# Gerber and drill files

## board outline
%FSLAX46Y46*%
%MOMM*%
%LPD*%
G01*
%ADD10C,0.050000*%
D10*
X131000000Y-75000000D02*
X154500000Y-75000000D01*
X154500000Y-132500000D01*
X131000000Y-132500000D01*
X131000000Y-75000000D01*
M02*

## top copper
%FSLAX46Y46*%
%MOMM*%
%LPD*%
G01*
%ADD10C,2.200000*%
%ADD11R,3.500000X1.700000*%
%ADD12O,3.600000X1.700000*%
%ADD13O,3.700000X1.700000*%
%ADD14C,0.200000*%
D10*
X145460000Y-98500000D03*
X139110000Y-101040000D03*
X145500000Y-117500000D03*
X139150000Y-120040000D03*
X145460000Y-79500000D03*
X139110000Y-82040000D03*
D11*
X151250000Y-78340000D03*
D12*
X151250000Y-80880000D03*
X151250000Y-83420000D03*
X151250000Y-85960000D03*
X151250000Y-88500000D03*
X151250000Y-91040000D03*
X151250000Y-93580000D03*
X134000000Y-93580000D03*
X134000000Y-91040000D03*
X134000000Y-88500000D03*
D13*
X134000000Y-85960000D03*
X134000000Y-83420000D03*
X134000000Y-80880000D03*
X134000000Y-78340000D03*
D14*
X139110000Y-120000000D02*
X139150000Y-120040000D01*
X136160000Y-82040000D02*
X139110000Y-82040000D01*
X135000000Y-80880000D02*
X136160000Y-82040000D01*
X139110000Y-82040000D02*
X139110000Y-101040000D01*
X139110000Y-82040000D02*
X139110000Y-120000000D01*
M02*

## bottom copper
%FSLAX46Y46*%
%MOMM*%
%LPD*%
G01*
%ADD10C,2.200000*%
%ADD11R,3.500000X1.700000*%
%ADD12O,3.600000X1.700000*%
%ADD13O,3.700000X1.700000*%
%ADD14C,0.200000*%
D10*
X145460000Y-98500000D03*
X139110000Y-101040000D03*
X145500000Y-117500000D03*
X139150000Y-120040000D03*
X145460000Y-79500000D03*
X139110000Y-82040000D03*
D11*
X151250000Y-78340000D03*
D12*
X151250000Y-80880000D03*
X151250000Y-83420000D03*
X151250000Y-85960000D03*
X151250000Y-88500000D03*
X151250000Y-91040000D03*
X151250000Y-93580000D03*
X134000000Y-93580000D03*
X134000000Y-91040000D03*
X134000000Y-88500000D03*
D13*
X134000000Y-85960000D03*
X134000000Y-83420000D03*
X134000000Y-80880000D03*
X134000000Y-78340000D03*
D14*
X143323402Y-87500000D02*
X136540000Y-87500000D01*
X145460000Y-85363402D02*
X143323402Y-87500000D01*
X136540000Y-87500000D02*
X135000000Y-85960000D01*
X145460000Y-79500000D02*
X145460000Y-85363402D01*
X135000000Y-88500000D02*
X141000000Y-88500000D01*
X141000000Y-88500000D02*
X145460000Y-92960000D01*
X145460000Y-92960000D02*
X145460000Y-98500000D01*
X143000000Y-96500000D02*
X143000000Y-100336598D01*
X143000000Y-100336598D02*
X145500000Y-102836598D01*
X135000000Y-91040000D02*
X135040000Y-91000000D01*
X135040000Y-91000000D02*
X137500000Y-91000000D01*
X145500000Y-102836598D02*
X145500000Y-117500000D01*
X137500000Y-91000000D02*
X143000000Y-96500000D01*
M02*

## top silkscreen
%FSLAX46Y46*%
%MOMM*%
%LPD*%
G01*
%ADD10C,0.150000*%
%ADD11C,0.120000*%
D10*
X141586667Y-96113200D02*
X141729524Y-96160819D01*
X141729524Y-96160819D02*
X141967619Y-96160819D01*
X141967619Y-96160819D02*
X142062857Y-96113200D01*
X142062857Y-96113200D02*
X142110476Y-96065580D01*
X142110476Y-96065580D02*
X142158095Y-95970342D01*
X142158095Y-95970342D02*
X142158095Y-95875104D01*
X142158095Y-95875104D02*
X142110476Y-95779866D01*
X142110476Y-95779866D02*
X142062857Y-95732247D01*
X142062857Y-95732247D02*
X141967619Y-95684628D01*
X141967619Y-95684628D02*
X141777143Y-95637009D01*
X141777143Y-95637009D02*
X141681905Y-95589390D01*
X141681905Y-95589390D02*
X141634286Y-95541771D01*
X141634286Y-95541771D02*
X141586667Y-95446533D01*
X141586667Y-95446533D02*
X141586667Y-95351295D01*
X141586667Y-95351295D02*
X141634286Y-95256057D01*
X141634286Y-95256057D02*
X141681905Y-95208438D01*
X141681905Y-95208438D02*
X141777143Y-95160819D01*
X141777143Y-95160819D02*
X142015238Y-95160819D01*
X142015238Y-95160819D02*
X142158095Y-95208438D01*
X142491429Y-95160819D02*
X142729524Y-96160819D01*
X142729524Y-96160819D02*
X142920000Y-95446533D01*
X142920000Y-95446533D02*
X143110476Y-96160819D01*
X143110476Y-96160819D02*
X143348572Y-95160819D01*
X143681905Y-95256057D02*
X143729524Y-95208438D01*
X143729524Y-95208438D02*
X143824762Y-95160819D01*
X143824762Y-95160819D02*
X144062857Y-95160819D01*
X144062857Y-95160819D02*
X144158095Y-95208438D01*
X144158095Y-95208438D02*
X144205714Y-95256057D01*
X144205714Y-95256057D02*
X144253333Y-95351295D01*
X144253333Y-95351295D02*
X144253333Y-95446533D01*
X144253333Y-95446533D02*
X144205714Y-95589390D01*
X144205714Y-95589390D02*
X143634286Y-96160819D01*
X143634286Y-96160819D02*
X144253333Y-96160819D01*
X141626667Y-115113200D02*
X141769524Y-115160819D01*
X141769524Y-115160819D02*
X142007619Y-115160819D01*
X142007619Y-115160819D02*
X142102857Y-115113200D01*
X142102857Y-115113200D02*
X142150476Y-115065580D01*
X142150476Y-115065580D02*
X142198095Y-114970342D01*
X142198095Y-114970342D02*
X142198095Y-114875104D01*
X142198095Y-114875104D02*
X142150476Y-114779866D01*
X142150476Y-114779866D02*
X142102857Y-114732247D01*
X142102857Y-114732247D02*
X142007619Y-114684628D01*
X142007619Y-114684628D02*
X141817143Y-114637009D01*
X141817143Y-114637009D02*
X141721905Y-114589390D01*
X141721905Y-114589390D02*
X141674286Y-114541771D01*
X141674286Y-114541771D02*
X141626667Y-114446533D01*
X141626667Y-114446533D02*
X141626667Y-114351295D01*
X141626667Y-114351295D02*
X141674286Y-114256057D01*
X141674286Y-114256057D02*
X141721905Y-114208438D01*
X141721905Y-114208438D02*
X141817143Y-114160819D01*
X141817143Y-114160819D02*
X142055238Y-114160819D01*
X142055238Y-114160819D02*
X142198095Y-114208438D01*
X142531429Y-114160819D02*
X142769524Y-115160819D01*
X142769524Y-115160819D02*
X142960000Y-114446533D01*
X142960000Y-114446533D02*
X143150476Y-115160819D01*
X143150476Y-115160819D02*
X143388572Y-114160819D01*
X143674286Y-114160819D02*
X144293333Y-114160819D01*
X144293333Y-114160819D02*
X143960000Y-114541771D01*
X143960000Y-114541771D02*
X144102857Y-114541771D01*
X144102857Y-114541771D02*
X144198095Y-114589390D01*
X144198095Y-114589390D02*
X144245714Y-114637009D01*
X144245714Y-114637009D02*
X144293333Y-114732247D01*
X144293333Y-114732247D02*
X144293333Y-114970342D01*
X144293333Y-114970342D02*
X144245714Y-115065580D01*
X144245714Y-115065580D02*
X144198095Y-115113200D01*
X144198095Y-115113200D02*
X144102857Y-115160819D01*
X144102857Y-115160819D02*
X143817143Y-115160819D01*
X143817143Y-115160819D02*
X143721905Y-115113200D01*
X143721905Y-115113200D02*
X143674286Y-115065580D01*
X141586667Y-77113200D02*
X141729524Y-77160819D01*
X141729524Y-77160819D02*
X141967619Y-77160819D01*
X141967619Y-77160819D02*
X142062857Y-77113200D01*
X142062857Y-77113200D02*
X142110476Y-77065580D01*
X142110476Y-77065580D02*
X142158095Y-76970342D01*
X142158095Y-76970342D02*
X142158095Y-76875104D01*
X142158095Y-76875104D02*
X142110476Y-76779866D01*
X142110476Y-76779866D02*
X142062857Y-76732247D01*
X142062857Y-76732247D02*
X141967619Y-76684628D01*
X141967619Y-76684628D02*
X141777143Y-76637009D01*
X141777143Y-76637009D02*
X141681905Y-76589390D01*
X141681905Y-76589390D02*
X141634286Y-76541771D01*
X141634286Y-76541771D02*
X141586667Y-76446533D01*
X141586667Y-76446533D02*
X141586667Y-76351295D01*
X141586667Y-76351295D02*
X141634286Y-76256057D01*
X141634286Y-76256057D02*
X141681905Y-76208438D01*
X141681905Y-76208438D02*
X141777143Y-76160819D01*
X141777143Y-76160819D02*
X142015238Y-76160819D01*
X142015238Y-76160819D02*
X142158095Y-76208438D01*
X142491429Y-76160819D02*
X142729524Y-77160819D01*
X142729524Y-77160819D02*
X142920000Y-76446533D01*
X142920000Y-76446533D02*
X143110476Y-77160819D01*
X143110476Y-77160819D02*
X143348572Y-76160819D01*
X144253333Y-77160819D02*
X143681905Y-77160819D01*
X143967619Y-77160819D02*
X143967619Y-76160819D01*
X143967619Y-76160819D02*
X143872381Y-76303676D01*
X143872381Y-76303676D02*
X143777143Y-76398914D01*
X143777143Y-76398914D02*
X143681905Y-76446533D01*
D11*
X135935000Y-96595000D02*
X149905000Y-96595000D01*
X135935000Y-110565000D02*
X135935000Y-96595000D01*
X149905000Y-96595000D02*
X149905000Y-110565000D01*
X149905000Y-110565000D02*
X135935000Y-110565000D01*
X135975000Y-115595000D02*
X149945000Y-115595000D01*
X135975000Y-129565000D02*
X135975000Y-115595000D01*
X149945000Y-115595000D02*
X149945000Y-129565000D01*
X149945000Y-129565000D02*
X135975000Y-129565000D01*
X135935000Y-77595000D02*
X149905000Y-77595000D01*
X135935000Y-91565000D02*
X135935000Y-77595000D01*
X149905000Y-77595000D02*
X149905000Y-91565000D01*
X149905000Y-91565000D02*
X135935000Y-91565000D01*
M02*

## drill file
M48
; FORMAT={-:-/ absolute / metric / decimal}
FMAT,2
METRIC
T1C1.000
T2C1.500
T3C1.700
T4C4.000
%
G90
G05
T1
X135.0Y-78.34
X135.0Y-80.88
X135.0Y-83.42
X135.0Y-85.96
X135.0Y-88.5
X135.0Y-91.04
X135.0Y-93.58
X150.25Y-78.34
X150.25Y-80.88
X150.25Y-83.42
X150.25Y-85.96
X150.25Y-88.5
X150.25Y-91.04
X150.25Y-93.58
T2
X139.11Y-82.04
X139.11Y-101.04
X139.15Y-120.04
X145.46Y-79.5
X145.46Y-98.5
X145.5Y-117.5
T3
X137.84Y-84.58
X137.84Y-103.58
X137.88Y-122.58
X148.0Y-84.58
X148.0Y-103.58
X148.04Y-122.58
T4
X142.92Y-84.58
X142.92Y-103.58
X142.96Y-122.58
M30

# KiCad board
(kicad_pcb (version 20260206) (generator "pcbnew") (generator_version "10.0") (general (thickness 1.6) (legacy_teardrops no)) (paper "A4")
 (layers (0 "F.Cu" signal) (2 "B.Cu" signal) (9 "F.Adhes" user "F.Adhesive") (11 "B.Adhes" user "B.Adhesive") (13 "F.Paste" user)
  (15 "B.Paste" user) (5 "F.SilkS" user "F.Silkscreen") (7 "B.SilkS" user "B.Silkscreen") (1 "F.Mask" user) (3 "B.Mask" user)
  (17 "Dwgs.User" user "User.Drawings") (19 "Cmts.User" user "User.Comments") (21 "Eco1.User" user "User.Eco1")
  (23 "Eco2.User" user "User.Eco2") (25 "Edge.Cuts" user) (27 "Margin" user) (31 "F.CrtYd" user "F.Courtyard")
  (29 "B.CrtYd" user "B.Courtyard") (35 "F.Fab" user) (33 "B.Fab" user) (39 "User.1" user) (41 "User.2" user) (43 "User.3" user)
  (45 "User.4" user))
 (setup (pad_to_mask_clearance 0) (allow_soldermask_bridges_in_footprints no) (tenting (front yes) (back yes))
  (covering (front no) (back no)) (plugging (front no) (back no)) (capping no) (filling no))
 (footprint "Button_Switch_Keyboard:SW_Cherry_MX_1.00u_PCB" (layer "F.Cu") (at 145.46 98.5)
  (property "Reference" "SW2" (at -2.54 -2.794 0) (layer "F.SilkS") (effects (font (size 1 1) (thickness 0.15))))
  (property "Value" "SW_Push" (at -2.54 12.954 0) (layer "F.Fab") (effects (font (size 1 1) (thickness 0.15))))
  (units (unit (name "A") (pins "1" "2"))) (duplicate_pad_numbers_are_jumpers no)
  (fp_line (start -9.525 -1.905) (end 4.445 -1.905) (stroke (width 0.12) (type solid)) (layer "F.SilkS"))
  (fp_line (start -9.525 12.065) (end -9.525 -1.905) (stroke (width 0.12) (type solid)) (layer "F.SilkS"))
  (fp_line (start 4.445 -1.905) (end 4.445 12.065) (stroke (width 0.12) (type solid)) (layer "F.SilkS"))
  (fp_line (start 4.445 12.065) (end -9.525 12.065) (stroke (width 0.12) (type solid)) (layer "F.SilkS"))
  (pad "" np_thru_hole circle (at -7.62 5.08) (size 1.7 1.7) (drill 1.7) (layers "*.Cu" "*.Mask"))
  (pad "" np_thru_hole circle (at -2.54 5.08) (size 4 4) (drill 4) (layers "*.Cu" "*.Mask"))
  (pad "" np_thru_hole circle (at 2.54 5.08) (size 1.7 1.7) (drill 1.7) (layers "*.Cu" "*.Mask"))
  (pad "1" thru_hole circle (at 0 0) (size 2.2 2.2) (drill 1.5) (layers "*.Cu" "*.Mask") (remove_unused_layers no)
   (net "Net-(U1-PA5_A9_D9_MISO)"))
  (pad "2" thru_hole circle (at -6.35 2.54) (size 2.2 2.2) (drill 1.5) (layers "*.Cu" "*.Mask") (remove_unused_layers no) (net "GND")))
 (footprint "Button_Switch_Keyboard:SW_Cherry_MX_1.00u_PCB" (layer "F.Cu") (at 145.5 117.5)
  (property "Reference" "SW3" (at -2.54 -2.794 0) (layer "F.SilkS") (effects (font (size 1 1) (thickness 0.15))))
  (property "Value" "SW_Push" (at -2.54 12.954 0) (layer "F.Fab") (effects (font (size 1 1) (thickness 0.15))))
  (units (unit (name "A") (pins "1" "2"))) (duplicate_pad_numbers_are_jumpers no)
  (fp_line (start -9.525 -1.905) (end 4.445 -1.905) (stroke (width 0.12) (type solid)) (layer "F.SilkS"))
  (fp_line (start -9.525 12.065) (end -9.525 -1.905) (stroke (width 0.12) (type solid)) (layer "F.SilkS"))
  (fp_line (start 4.445 -1.905) (end 4.445 12.065) (stroke (width 0.12) (type solid)) (layer "F.SilkS"))
  (fp_line (start 4.445 12.065) (end -9.525 12.065) (stroke (width 0.12) (type solid)) (layer "F.SilkS"))
  (pad "" np_thru_hole circle (at -7.62 5.08) (size 1.7 1.7) (drill 1.7) (layers "*.Cu" "*.Mask"))
  (pad "" np_thru_hole circle (at -2.54 5.08) (size 4 4) (drill 4) (layers "*.Cu" "*.Mask"))
  (pad "" np_thru_hole circle (at 2.54 5.08) (size 1.7 1.7) (drill 1.7) (layers "*.Cu" "*.Mask"))
  (pad "1" thru_hole circle (at 0 0) (size 2.2 2.2) (drill 1.5) (layers "*.Cu" "*.Mask") (remove_unused_layers no)
   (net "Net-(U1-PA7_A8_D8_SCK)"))
  (pad "2" thru_hole circle (at -6.35 2.54) (size 2.2 2.2) (drill 1.5) (layers "*.Cu" "*.Mask") (remove_unused_layers no) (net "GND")))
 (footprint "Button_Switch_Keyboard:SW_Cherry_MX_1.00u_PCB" (layer "F.Cu") (at 145.46 79.5)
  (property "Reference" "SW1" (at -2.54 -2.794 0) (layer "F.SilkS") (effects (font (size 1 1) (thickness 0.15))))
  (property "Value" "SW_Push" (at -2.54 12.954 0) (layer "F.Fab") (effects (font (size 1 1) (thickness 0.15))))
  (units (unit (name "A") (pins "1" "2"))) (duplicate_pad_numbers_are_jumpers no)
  (fp_line (start -9.525 -1.905) (end 4.445 -1.905) (stroke (width 0.12) (type solid)) (layer "F.SilkS"))
  (fp_line (start -9.525 12.065) (end -9.525 -1.905) (stroke (width 0.12) (type solid)) (layer "F.SilkS"))
  (fp_line (start 4.445 -1.905) (end 4.445 12.065) (stroke (width 0.12) (type solid)) (layer "F.SilkS"))
  (fp_line (start 4.445 12.065) (end -9.525 12.065) (stroke (width 0.12) (type solid)) (layer "F.SilkS"))
  (pad "" np_thru_hole circle (at -7.62 5.08) (size 1.7 1.7) (drill 1.7) (layers "*.Cu" "*.Mask"))
  (pad "" np_thru_hole circle (at -2.54 5.08) (size 4 4) (drill 4) (layers "*.Cu" "*.Mask"))
  (pad "" np_thru_hole circle (at 2.54 5.08) (size 1.7 1.7) (drill 1.7) (layers "*.Cu" "*.Mask"))
  (pad "1" thru_hole circle (at 0 0) (size 2.2 2.2) (drill 1.5) (layers "*.Cu" "*.Mask") (remove_unused_layers no)
   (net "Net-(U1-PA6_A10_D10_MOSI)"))
  (pad "2" thru_hole circle (at -6.35 2.54) (size 2.2 2.2) (drill 1.5) (layers "*.Cu" "*.Mask") (remove_unused_layers no) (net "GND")))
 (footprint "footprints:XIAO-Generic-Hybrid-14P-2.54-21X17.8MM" (layer "B.Cu") (at 142.625 85.96 180)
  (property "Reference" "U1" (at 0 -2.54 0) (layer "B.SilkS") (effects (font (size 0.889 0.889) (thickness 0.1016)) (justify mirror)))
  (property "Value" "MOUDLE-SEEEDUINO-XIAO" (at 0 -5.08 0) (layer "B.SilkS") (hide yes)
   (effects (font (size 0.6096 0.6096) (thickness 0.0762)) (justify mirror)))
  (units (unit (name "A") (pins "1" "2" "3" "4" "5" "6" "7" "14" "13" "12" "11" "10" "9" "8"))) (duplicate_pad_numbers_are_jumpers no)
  (pad "1" thru_hole rect (at -7.625 7.62 180) (size 3.5 1.7) (drill 1 (offset -1 0)) (layers "*.Cu" "*.Mask") (remove_unused_layers no)
   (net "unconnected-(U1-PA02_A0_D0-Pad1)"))
  (pad "2" thru_hole oval (at -7.625 5.08 180) (size 3.6 1.7) (drill 1 (offset -1 0)) (layers "*.Cu" "*.Mask") (remove_unused_layers no)
   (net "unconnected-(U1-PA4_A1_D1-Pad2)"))
  (pad "3" thru_hole oval (at -7.625 2.54 180) (size 3.6 1.7) (drill 1 (offset -1 0)) (layers "*.Cu" "*.Mask") (remove_unused_layers no)
   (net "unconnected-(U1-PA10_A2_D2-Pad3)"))
  (pad "4" thru_hole oval (at -7.625 0 180) (size 3.6 1.7) (drill 1 (offset -1 0)) (layers "*.Cu" "*.Mask") (remove_unused_layers no)
   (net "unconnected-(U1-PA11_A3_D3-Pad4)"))
  (pad "5" thru_hole oval (at -7.625 -2.54 180) (size 3.6 1.7) (drill 1 (offset -1 0)) (layers "*.Cu" "*.Mask") (remove_unused_layers no)
   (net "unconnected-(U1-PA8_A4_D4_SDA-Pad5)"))
  (pad "6" thru_hole oval (at -7.625 -5.08) (size 3.6 1.7) (drill 1 (offset 1 0)) (layers "*.Cu" "*.Mask") (remove_unused_layers no)
   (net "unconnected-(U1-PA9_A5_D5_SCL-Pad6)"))
  (pad "7" thru_hole oval (at -7.625 -7.62 180) (size 3.6 1.7) (drill 1 (offset -1 0)) (layers "*.Cu" "*.Mask") (remove_unused_layers no)
   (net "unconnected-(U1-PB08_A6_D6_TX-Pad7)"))
  (pad "8" thru_hole oval (at 7.625 -7.62 180) (size 3.6 1.7) (drill 1 (offset 1 0)) (layers "*.Cu" "*.Mask") (remove_unused_layers no)
   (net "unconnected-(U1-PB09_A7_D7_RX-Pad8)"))
  (pad "9" thru_hole oval (at 7.625 -5.08 180) (size 3.6 1.7) (drill 1 (offset 1 0)) (layers "*.Cu" "*.Mask") (remove_unused_layers no)
   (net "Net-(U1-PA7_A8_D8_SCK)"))
  (pad "10" thru_hole oval (at 7.625 -2.54 180) (size 3.6 1.7) (drill 1 (offset 1 0)) (layers "*.Cu" "*.Mask") (remove_unused_layers no)
   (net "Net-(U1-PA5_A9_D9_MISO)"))
  (pad "11" thru_hole oval (at 7.625 0 180) (size 3.7 1.7) (drill 1 (offset 1 0)) (layers "*.Cu" "*.Mask") (remove_unused_layers no)
   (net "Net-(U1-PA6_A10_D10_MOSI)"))
  (pad "12" thru_hole oval (at 7.625 2.54 180) (size 3.7 1.7) (drill 1 (offset 1 0)) (layers "*.Cu" "*.Mask") (remove_unused_layers no)
   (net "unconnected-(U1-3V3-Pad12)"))
  (pad "13" thru_hole oval (at 7.625 5.08 180) (size 3.7 1.7) (drill 1 (offset 1 0)) (layers "*.Cu" "*.Mask") (remove_unused_layers no)
   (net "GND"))
  (pad "14" thru_hole oval (at 7.625 7.62 180) (size 3.7 1.7) (drill 1 (offset 1 0)) (layers "*.Cu" "*.Mask") (remove_unused_layers no)
   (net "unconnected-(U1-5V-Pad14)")))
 (gr_rect (start 131 75) (end 154.5 132.5) (stroke (width 0.05) (type default)) (fill no) (layer "Edge.Cuts"))
 (segment (start 143.323402 87.5) (end 136.54 87.5) (width 0.2) (layer "B.Cu") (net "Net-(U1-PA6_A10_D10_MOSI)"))
 (segment (start 145.46 85.363402) (end 143.323402 87.5) (width 0.2) (layer "B.Cu") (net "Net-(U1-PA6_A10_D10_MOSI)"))
 (segment (start 136.54 87.5) (end 135 85.96) (width 0.2) (layer "B.Cu") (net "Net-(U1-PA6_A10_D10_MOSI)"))
 (segment (start 145.46 79.5) (end 145.46 85.363402) (width 0.2) (layer "B.Cu") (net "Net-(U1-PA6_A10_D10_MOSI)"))
 (segment (start 139.11 120) (end 139.15 120.04) (width 0.2) (layer "F.Cu") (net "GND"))
 (segment (start 136.16 82.04) (end 139.11 82.04) (width 0.2) (layer "F.Cu") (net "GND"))
 (segment (start 135 80.88) (end 136.16 82.04) (width 0.2) (layer "F.Cu") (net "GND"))
 (segment (start 139.11 82.04) (end 139.11 101.04) (width 0.2) (layer "F.Cu") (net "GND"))
 (segment (start 139.11 82.04) (end 139.11 120) (width 0.2) (layer "F.Cu") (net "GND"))
 (segment (start 135 88.5) (end 141 88.5) (width 0.2) (layer "B.Cu") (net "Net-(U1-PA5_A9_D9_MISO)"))
 (segment (start 141 88.5) (end 145.46 92.96) (width 0.2) (layer "B.Cu") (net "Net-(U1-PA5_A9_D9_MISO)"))
 (segment (start 145.46 92.96) (end 145.46 98.5) (width 0.2) (layer "B.Cu") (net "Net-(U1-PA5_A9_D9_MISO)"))
 (segment (start 143 96.5) (end 143 100.336598) (width 0.2) (layer "B.Cu") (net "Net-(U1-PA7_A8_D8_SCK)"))
 (segment (start 143 100.336598) (end 145.5 102.836598) (width 0.2) (layer "B.Cu") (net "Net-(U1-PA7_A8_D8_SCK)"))
 (segment (start 135 91.04) (end 135.04 91) (width 0.2) (layer "B.Cu") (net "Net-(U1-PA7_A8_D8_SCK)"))
 (segment (start 135.04 91) (end 137.5 91) (width 0.2) (layer "B.Cu") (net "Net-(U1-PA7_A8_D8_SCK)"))
 (segment (start 145.5 102.836598) (end 145.5 117.5) (width 0.2) (layer "B.Cu") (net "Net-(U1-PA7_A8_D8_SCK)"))
 (segment (start 137.5 91) (end 143 96.5) (width 0.2) (layer "B.Cu") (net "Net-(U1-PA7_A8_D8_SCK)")))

